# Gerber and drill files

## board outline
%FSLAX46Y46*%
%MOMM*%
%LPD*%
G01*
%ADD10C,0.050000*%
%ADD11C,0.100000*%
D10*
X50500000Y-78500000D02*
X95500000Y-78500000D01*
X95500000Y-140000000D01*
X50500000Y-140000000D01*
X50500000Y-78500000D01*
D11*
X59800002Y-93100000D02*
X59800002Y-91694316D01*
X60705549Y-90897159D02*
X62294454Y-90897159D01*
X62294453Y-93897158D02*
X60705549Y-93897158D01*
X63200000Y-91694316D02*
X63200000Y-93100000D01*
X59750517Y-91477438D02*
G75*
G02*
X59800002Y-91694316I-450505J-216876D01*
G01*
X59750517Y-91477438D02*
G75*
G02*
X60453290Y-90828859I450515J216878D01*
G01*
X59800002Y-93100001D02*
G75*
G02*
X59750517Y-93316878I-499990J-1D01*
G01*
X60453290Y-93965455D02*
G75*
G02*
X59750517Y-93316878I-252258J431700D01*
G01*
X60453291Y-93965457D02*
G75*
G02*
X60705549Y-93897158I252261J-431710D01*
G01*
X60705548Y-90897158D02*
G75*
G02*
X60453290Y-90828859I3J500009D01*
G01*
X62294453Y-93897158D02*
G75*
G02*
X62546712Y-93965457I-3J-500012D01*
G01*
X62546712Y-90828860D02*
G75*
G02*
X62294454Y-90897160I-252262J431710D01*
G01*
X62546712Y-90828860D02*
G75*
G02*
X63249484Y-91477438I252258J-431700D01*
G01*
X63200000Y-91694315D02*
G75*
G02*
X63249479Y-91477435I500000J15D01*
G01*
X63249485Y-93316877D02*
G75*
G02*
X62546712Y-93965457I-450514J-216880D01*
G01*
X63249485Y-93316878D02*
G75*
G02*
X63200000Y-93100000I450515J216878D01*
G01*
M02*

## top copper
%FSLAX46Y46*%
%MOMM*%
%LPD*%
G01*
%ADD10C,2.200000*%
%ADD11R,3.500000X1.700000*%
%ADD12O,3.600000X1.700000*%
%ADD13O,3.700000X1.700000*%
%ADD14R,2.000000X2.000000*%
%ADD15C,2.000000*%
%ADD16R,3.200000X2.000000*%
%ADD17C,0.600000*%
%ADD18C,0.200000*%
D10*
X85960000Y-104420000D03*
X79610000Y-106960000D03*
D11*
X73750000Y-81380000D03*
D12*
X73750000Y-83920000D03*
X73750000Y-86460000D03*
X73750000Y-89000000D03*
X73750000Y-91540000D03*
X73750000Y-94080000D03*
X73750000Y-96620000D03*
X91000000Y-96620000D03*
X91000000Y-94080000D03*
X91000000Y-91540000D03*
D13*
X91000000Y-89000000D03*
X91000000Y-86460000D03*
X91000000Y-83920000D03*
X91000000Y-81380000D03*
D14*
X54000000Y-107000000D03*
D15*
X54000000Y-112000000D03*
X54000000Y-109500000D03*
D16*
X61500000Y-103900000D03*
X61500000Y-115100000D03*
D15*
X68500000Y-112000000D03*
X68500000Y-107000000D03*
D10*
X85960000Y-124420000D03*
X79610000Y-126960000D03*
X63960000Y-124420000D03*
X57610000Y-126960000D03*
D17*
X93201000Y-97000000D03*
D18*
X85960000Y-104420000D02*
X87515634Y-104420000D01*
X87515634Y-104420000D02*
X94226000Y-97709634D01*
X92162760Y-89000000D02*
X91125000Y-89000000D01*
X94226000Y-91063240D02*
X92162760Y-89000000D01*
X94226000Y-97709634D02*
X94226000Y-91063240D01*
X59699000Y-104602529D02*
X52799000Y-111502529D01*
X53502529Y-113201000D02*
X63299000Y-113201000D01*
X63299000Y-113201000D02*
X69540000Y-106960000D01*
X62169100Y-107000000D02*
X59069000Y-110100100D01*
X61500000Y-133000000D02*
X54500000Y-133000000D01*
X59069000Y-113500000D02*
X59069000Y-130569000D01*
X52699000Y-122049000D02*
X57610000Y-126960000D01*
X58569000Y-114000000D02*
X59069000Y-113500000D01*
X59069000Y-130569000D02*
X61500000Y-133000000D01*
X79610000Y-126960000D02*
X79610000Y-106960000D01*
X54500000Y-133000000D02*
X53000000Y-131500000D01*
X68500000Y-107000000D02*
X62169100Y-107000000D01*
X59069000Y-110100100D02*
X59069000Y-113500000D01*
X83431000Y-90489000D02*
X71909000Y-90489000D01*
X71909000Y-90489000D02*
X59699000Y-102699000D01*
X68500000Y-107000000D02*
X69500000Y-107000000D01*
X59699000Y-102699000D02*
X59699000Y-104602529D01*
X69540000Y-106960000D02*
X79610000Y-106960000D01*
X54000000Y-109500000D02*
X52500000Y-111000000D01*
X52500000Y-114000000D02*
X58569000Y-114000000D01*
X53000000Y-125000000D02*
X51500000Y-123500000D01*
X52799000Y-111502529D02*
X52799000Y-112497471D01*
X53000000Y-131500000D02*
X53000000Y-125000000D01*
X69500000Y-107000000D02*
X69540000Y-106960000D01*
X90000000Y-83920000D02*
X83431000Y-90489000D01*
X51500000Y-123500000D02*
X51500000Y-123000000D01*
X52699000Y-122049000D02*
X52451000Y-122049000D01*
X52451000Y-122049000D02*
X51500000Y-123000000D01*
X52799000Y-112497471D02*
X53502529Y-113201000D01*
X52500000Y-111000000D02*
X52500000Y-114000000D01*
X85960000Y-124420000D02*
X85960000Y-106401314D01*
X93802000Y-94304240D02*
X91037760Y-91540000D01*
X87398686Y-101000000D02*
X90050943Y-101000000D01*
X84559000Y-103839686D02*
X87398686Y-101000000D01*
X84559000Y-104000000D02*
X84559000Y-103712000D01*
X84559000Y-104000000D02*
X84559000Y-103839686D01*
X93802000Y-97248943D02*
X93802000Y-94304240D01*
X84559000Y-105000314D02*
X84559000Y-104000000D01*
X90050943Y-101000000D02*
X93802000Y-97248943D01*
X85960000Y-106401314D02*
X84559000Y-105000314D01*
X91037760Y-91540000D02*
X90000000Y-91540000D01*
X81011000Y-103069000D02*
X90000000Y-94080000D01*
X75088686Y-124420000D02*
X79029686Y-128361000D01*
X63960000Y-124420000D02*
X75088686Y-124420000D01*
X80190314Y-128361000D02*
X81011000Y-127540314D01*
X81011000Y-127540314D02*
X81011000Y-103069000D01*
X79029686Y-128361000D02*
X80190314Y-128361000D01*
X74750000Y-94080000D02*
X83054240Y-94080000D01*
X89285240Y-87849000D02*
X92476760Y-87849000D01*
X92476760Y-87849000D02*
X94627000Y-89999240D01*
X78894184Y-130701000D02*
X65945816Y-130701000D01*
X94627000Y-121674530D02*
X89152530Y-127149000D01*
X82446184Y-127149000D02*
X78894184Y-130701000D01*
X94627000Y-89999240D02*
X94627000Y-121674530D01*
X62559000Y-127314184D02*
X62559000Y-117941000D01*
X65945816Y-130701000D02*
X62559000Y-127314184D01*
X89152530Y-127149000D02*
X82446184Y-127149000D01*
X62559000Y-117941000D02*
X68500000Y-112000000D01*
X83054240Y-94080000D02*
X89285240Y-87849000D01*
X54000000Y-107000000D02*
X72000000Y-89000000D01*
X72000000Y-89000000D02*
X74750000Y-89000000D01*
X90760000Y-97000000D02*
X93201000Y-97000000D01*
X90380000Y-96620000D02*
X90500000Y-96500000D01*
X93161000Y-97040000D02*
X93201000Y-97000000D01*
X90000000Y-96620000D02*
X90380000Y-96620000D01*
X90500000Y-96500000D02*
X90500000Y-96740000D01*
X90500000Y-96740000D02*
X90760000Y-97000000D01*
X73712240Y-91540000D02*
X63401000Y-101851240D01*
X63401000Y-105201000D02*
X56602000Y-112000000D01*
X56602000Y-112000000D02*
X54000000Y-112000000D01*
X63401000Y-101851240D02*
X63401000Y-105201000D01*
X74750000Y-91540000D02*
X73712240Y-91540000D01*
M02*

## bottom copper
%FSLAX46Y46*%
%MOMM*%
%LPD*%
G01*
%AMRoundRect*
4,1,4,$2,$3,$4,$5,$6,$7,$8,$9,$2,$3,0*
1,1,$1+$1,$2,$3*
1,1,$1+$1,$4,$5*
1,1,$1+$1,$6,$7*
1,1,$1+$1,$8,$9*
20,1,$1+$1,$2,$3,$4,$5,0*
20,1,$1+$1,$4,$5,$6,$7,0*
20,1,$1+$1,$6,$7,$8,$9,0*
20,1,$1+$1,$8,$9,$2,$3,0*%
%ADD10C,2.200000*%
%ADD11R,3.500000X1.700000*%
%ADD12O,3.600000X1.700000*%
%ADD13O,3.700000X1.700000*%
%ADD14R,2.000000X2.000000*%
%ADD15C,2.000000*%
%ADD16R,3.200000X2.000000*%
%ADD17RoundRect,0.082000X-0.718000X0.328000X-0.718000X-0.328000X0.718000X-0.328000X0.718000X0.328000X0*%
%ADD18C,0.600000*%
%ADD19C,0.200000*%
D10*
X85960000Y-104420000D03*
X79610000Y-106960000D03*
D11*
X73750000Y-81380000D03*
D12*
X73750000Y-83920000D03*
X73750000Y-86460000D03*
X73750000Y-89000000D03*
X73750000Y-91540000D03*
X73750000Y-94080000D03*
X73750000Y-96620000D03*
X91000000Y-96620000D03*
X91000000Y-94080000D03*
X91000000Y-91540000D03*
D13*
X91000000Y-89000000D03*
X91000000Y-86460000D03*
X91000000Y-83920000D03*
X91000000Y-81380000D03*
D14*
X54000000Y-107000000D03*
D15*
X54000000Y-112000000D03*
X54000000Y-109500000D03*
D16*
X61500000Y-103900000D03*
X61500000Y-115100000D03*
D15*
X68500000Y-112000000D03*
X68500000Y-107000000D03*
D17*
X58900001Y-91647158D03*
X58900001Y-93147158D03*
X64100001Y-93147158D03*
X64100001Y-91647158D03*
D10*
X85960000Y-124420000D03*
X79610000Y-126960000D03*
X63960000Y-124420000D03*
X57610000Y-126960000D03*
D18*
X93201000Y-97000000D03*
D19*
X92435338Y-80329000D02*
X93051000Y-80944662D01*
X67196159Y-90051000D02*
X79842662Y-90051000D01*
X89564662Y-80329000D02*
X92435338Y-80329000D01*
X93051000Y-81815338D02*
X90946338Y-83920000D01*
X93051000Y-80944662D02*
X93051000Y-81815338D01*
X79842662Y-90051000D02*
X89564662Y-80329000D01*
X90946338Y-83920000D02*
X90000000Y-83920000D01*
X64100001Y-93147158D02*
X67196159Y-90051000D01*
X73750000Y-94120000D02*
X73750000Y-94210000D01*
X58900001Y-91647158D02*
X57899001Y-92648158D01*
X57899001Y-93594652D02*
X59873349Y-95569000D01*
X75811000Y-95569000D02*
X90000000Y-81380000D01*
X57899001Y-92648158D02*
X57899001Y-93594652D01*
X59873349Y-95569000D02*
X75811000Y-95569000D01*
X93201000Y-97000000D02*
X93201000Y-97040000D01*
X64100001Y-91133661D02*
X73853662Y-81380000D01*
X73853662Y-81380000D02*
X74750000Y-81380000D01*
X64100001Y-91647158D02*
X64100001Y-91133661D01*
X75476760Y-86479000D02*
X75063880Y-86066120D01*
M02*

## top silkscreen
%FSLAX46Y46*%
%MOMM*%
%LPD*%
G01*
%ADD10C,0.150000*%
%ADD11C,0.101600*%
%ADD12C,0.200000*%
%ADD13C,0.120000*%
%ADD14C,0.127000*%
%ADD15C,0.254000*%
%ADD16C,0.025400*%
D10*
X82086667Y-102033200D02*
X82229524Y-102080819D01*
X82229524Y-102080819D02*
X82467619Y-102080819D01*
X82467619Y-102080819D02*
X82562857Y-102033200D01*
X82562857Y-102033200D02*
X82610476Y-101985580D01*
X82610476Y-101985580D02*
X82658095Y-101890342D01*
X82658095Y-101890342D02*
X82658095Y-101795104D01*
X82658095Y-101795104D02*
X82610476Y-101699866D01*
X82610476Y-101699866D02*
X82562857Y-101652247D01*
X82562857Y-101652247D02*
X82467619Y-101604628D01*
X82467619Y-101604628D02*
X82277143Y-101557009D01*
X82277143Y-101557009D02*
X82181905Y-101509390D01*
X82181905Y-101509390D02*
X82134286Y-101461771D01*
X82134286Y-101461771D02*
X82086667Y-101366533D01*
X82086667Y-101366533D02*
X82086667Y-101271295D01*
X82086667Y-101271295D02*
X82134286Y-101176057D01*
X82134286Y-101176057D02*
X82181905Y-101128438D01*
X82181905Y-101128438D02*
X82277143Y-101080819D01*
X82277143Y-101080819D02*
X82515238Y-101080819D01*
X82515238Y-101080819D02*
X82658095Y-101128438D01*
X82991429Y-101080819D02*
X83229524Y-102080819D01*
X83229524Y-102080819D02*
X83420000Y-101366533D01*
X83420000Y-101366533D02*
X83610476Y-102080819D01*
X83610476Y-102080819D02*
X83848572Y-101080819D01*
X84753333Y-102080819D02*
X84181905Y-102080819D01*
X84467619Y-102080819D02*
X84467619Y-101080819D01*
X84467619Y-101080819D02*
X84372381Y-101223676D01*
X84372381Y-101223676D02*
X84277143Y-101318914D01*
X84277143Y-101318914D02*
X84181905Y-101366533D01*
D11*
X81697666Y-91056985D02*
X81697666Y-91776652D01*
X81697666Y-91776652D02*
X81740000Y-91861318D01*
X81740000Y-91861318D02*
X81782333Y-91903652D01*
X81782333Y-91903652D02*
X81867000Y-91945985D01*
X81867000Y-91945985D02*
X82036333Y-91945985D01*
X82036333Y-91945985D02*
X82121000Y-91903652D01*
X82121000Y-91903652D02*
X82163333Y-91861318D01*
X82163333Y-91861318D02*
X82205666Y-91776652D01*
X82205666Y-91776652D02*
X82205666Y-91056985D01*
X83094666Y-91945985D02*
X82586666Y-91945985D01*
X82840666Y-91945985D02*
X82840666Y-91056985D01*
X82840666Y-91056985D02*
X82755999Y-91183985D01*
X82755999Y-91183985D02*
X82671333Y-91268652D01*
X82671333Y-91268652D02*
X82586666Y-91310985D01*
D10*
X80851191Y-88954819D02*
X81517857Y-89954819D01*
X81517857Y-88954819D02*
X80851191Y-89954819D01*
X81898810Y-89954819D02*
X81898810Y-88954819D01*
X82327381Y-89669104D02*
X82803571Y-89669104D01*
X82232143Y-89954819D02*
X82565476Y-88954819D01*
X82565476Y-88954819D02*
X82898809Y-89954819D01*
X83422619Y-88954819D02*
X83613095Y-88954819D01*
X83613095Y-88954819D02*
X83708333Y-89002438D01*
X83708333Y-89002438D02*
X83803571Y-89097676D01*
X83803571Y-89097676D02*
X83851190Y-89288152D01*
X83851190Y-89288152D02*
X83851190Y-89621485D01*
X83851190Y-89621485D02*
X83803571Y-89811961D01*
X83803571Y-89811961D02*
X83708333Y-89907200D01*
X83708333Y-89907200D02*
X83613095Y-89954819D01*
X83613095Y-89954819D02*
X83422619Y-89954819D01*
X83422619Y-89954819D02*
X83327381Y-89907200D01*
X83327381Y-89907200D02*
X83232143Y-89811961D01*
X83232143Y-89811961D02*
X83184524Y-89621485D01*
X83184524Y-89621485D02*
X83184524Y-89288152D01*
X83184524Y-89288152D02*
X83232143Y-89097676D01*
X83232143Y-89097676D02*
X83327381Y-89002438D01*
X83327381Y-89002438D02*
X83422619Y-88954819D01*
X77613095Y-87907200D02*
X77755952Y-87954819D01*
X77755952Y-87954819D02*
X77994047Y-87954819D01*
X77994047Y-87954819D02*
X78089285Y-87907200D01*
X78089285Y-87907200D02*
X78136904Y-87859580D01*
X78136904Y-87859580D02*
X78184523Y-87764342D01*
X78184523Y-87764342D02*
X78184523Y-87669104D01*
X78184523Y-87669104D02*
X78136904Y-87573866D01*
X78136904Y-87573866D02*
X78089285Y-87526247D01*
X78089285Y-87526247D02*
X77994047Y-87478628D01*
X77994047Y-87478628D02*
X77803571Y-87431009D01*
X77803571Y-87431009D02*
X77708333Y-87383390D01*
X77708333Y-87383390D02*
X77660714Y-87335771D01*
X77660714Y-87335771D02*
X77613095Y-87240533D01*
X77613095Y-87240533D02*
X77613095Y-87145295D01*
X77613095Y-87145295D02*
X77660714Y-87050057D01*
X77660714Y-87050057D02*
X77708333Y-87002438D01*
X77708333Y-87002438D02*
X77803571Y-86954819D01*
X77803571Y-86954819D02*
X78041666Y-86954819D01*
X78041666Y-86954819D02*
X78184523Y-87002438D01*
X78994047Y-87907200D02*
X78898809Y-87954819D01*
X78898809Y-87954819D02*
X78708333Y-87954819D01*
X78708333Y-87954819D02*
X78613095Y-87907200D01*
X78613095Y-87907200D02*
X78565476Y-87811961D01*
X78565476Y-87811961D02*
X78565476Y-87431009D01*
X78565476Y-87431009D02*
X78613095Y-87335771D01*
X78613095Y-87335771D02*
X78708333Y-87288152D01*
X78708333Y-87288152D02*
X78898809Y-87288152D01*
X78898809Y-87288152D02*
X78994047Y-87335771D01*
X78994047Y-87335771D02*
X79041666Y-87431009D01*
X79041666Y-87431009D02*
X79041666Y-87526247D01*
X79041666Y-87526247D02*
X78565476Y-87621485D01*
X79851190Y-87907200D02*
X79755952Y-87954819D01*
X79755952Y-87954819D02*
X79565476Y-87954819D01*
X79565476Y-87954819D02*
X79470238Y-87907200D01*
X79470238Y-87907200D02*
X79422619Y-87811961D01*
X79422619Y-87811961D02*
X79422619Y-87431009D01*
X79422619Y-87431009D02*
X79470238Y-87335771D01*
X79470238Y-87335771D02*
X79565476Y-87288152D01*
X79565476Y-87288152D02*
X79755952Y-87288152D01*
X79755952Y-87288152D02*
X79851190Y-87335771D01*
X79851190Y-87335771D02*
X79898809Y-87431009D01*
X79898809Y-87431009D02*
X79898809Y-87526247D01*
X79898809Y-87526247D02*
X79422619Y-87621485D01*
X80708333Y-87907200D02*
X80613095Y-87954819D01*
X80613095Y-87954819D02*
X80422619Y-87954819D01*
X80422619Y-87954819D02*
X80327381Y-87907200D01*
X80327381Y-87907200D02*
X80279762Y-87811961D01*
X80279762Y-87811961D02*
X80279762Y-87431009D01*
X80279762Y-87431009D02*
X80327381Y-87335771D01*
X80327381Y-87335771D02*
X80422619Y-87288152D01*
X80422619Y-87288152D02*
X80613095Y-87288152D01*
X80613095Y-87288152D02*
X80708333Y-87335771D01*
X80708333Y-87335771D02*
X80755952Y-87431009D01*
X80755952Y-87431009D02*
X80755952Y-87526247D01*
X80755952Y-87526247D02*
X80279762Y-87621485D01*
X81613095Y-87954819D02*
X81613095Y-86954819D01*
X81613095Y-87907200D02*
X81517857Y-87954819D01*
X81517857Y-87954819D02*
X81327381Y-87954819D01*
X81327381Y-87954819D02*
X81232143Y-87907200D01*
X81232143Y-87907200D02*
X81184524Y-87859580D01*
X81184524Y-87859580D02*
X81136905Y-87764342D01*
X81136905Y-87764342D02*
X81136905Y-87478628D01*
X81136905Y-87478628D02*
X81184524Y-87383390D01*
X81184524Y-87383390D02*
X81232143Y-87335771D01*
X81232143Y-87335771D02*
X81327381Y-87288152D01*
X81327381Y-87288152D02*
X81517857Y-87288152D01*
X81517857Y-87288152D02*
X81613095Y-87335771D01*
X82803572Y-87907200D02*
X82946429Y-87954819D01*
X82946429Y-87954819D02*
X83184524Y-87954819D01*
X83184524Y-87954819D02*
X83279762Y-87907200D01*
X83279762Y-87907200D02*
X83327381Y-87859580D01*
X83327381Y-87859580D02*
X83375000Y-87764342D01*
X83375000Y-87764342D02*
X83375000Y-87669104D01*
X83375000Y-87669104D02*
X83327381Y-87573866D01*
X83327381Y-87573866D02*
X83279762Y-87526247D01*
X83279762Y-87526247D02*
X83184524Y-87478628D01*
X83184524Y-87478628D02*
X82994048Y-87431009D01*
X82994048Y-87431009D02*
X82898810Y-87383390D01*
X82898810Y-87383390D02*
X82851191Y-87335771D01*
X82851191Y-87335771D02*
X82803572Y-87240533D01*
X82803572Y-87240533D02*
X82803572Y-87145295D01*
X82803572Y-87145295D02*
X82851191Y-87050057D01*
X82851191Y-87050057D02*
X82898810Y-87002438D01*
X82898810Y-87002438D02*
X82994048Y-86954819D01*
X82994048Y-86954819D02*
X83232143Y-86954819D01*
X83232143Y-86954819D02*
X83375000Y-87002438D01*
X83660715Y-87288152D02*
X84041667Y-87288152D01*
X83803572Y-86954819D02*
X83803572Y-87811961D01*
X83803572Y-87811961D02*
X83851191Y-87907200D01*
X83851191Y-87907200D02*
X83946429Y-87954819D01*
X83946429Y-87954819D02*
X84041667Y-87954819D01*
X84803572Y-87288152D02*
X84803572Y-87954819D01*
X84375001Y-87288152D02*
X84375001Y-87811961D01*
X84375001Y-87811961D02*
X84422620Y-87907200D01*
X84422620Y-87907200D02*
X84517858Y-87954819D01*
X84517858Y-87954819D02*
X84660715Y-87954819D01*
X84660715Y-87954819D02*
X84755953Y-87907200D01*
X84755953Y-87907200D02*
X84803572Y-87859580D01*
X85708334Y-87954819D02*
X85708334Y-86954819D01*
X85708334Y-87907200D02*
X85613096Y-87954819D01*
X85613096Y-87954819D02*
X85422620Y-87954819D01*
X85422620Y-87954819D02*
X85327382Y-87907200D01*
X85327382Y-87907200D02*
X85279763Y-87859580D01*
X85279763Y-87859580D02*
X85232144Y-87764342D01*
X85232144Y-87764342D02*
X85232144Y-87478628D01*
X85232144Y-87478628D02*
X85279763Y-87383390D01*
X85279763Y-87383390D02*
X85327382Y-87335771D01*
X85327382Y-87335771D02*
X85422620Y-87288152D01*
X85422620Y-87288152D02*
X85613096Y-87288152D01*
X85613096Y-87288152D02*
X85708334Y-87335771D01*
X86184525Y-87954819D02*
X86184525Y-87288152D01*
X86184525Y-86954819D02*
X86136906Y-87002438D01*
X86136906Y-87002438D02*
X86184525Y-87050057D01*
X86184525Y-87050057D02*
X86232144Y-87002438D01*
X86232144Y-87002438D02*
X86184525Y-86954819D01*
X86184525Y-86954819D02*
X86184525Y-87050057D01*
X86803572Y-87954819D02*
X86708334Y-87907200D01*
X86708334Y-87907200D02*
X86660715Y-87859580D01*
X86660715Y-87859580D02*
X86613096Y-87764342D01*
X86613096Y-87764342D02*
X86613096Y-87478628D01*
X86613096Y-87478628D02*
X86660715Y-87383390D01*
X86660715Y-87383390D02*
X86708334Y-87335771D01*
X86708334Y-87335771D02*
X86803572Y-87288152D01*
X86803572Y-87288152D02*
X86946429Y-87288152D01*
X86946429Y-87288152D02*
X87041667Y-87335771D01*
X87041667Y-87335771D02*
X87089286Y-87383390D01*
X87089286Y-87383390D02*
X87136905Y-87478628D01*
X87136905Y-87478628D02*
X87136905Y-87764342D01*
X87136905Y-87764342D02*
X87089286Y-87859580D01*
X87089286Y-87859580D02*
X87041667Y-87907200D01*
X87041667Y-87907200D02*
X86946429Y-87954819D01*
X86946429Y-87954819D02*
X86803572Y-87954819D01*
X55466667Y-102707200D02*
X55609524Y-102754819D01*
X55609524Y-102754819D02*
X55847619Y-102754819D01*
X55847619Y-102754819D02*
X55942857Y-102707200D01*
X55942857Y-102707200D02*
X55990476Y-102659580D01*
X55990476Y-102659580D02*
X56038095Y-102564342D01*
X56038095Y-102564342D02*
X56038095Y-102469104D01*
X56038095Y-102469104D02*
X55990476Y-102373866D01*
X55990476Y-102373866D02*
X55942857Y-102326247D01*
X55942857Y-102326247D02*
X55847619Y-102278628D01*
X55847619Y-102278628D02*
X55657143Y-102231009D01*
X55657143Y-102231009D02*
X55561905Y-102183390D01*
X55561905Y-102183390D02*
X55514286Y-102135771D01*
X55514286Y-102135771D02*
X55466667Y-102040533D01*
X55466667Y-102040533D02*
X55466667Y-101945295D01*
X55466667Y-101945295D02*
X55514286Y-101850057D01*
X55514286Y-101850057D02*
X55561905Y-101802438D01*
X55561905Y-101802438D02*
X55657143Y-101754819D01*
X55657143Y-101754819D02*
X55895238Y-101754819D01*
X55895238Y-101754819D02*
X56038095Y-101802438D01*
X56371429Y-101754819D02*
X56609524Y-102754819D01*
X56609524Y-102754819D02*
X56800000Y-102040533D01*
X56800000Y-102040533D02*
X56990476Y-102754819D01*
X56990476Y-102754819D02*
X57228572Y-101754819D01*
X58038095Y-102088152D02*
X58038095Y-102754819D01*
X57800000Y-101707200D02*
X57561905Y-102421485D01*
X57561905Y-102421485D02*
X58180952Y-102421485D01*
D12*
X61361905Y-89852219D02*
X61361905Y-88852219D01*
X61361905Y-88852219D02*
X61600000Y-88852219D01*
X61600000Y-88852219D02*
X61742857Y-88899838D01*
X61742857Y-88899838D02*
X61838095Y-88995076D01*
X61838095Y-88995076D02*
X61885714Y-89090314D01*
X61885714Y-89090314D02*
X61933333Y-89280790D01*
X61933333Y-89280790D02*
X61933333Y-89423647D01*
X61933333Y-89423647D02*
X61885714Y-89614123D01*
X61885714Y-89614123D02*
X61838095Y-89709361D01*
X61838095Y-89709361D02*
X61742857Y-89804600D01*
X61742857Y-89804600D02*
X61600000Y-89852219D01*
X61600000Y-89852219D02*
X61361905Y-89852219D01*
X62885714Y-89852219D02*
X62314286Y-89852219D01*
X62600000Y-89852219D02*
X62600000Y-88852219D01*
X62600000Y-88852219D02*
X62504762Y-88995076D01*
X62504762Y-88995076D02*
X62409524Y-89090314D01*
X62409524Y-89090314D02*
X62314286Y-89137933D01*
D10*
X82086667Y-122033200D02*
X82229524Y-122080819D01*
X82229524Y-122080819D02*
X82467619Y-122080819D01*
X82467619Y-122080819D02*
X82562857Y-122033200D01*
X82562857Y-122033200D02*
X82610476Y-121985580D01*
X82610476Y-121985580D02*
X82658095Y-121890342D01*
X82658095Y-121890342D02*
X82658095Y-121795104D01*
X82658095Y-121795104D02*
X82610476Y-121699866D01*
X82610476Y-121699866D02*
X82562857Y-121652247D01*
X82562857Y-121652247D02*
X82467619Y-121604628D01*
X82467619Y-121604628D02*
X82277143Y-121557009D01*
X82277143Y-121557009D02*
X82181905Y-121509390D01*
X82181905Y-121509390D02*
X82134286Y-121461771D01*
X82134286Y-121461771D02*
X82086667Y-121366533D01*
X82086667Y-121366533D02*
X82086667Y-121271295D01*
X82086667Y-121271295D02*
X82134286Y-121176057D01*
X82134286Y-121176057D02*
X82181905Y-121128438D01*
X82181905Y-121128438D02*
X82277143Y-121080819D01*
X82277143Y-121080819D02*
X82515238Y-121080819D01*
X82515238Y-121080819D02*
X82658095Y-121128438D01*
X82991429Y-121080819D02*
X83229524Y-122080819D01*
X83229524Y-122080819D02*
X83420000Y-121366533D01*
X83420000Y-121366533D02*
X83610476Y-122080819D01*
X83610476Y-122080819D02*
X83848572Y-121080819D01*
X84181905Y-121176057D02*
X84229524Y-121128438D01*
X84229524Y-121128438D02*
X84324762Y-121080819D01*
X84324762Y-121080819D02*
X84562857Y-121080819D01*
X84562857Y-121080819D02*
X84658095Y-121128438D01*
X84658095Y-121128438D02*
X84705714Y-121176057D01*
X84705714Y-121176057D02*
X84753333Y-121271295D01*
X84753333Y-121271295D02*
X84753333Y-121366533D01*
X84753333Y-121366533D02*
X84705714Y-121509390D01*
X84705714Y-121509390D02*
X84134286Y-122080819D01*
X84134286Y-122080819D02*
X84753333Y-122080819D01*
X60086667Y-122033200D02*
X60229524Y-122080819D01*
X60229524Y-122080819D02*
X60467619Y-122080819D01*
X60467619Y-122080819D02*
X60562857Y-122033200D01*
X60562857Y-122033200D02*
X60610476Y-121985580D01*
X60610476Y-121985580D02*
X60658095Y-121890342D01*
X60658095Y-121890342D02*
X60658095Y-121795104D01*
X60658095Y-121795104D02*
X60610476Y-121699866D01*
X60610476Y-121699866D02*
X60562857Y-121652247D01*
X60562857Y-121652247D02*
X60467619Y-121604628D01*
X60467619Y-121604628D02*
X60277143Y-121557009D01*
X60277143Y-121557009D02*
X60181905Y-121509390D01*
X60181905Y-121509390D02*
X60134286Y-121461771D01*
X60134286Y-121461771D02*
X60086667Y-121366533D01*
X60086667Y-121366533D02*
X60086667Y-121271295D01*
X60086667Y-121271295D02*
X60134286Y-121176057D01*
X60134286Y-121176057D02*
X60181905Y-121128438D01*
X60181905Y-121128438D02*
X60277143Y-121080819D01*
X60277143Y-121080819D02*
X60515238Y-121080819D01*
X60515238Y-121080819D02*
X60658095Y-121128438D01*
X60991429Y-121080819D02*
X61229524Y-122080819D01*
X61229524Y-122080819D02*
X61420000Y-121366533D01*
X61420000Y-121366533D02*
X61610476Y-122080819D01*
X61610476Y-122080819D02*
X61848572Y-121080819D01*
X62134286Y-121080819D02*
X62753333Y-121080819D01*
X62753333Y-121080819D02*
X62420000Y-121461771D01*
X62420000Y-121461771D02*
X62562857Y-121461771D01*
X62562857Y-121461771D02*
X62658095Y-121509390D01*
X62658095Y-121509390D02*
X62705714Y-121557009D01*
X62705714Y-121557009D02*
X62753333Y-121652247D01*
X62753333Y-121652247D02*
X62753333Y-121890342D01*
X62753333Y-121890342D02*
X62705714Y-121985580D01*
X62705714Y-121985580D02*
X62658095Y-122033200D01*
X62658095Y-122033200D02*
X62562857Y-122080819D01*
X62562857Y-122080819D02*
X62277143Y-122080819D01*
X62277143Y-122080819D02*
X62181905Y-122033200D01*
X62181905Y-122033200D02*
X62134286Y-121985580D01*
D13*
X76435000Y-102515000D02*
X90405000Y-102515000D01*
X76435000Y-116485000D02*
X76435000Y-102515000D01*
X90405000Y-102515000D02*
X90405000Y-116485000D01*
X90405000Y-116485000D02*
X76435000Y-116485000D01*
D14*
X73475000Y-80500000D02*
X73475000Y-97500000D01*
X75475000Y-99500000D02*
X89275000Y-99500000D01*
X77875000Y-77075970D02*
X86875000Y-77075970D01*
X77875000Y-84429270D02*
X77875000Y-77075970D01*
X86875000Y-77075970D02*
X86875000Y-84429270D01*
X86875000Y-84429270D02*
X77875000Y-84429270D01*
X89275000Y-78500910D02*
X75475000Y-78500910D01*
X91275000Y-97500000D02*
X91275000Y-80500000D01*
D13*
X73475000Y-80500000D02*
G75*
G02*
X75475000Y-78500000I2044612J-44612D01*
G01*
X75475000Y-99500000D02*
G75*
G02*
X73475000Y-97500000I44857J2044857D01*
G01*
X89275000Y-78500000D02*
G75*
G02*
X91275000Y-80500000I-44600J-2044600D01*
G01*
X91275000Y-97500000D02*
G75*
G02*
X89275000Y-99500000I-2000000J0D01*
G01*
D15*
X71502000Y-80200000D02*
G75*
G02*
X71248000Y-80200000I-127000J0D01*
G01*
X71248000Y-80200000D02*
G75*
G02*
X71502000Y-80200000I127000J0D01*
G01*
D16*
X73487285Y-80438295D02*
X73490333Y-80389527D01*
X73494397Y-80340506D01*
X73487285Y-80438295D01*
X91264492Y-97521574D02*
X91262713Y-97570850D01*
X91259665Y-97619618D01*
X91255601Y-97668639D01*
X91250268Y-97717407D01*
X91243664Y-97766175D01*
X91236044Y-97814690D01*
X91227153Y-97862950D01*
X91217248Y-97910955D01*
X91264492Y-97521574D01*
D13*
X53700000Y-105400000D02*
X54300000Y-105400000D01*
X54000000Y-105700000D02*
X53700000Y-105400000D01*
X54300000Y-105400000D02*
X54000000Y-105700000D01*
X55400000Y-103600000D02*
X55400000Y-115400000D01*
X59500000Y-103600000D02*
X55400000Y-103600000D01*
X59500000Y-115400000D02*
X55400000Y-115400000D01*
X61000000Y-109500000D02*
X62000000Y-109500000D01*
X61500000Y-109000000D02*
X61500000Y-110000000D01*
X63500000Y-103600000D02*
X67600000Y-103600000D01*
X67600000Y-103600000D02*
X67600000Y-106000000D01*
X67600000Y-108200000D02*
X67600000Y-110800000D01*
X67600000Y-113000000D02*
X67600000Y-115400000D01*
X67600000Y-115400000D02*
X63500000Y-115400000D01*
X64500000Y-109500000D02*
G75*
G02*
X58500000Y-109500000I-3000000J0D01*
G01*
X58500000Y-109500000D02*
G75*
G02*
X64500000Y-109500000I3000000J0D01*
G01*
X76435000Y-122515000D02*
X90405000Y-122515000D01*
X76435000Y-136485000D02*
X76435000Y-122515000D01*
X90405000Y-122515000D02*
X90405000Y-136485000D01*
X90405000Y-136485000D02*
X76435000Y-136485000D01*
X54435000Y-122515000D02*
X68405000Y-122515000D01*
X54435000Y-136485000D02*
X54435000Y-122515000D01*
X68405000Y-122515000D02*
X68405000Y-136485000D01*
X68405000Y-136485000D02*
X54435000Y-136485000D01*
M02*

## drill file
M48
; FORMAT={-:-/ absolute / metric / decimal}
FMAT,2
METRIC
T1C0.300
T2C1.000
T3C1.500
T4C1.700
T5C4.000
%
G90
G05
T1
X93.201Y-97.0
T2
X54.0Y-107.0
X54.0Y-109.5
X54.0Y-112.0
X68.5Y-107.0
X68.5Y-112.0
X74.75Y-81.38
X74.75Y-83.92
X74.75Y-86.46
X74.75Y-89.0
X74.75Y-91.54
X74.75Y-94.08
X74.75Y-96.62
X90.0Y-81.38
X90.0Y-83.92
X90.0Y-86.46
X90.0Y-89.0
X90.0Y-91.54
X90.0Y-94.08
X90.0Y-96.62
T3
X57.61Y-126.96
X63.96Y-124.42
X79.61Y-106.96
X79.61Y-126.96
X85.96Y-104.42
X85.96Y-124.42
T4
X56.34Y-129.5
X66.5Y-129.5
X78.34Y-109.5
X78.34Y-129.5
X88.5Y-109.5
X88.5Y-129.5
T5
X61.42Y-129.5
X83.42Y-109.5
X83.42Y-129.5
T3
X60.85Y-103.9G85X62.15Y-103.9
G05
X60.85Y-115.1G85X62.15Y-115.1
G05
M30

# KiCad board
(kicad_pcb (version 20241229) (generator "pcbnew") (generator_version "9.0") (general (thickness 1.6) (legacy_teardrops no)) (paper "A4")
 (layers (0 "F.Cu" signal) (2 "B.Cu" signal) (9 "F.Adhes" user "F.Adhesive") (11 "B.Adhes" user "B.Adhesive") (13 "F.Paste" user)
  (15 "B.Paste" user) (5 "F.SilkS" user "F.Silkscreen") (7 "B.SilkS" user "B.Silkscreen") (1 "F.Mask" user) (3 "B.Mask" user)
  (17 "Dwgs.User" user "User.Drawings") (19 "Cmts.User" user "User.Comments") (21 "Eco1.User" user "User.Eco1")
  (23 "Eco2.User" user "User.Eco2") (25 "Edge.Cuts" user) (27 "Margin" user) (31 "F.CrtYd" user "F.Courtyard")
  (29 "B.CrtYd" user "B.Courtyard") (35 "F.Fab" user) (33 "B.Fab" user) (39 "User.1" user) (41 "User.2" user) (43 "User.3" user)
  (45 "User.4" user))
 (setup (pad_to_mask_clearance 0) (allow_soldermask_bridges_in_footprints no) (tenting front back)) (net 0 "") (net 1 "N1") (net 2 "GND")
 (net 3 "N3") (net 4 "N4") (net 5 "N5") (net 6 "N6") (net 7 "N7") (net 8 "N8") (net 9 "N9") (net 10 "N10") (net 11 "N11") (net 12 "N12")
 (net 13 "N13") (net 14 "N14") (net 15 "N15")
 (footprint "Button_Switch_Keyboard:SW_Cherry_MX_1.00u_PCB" (layer "F.Cu") (at 85.96 104.42)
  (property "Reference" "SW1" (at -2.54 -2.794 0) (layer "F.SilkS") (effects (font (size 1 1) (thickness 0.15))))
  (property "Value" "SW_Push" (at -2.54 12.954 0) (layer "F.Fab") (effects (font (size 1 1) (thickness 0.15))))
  (fp_line (start -9.525 -1.905) (end 4.445 -1.905) (stroke (width 0.12) (type solid)) (layer "F.SilkS"))
  (fp_line (start -9.525 12.065) (end -9.525 -1.905) (stroke (width 0.12) (type solid)) (layer "F.SilkS"))
  (fp_line (start 4.445 -1.905) (end 4.445 12.065) (stroke (width 0.12) (type solid)) (layer "F.SilkS"))
  (fp_line (start 4.445 12.065) (end -9.525 12.065) (stroke (width 0.12) (type solid)) (layer "F.SilkS"))
  (pad "" np_thru_hole circle (at -7.62 5.08) (size 1.7 1.7) (drill 1.7) (layers "*.Cu" "*.Mask"))
  (pad "" np_thru_hole circle (at -2.54 5.08) (size 4 4) (drill 4) (layers "*.Cu" "*.Mask"))
  (pad "" np_thru_hole circle (at 2.54 5.08) (size 1.7 1.7) (drill 1.7) (layers "*.Cu" "*.Mask"))
  (pad "1" thru_hole circle (at 0 0) (size 2.2 2.2) (drill 1.5) (layers "*.Cu" "*.Mask") (remove_unused_layers no) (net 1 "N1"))
  (pad "2" thru_hole circle (at -6.35 2.54) (size 2.2 2.2) (drill 1.5) (layers "*.Cu" "*.Mask") (remove_unused_layers no) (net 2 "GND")))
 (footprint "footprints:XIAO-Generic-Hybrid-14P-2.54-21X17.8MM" (layer "F.Cu") (at 82.375 89)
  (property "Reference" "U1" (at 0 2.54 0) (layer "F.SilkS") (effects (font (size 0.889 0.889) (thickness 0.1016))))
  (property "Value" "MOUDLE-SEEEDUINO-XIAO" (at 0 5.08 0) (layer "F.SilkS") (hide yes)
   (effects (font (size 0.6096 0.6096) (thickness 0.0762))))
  (fp_line (start -8.9 -8.5) (end -8.9 8.5) (stroke (width 0.127) (type solid)) (layer "F.SilkS"))
  (fp_line (start -6.9 10.5) (end 6.9 10.5) (stroke (width 0.127) (type solid)) (layer "F.SilkS"))
  (fp_line (start -4.5 -11.92403) (end 4.5 -11.92403) (stroke (width 0.127) (type solid)) (layer "F.SilkS"))
  (fp_line (start -4.5 -4.57073) (end -4.5 -11.92403) (stroke (width 0.127) (type solid)) (layer "F.SilkS"))
  (fp_line (start 4.5 -11.92403) (end 4.5 -4.57073) (stroke (width 0.127) (type solid)) (layer "F.SilkS"))
  (fp_line (start 4.5 -4.57073) (end -4.5 -4.57073) (stroke (width 0.127) (type solid)) (layer "F.SilkS"))
  (fp_line (start 6.9 -10.49909) (end -6.9 -10.49909) (stroke (width 0.127) (type solid)) (layer "F.SilkS"))
  (fp_line (start 8.9 8.5) (end 8.9 -8.5) (stroke (width 0.127) (type solid)) (layer "F.SilkS"))
  (fp_arc (start -8.9 -8.5) (mid -8.301491 -9.901491) (end -6.9 -10.5) (stroke (width 0.12) (type solid)) (layer "F.SilkS"))
  (fp_arc (start -6.9 10.5) (mid -8.301423 9.901423) (end -8.9 8.5) (stroke (width 0.12) (type solid)) (layer "F.SilkS"))
  (fp_arc (start 6.9 -10.5) (mid 8.301492 -9.901492) (end 8.9 -8.5) (stroke (width 0.12) (type solid)) (layer "F.SilkS"))
  (fp_arc (start 8.9 8.5) (mid 8.314214 9.914214) (end 6.9 10.5) (stroke (width 0.12) (type solid)) (layer "F.SilkS"))
  (fp_circle (center -11 -8.8) (end -11 -9.054) (stroke (width 0) (type solid)) (fill yes) (layer "F.SilkS"))
  (fp_poly
   (pts (xy -8.887715 -8.561705) (xy -8.884667 -8.610473) (xy -8.880603 -8.659494)) (stroke (width 0.0254) (type solid)) (fill no)
   (layer "F.SilkS"))
  (fp_poly
   (pts (xy 8.889492 8.521574) (xy 8.887713 8.57085) (xy 8.884665 8.619618) (xy 8.880601 8.668639) (xy 8.875268 8.717407)
    (xy 8.868664 8.766175) (xy 8.861044 8.81469) (xy 8.852153 8.86295) (xy 8.842248 8.910955))
   (stroke (width 0.0254) (type solid)) (fill no) (layer "F.SilkS"))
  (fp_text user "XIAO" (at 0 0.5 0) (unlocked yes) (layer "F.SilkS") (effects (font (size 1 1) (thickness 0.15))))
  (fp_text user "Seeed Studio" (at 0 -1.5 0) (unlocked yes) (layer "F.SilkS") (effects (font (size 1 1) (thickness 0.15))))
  (pad "1" thru_hole rect (at -7.625 -7.62) (size 3.5 1.7) (drill 1 (offset -1 0)) (layers "*.Cu" "*.Mask") (remove_unused_layers no)
   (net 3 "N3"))
  (pad "2" thru_hole oval (at -7.625 -5.08) (size 3.6 1.7) (drill 1 (offset -1 0)) (layers "*.Cu" "*.Mask") (remove_unused_layers no)
   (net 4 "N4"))
  (pad "3" thru_hole oval (at -7.625 -2.54) (size 3.6 1.7) (drill 1 (offset -1 0)) (layers "*.Cu" "*.Mask") (remove_unused_layers no)
   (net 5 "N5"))
  (pad "4" thru_hole oval (at -7.625 0) (size 3.6 1.7) (drill 1 (offset -1 0)) (layers "*.Cu" "*.Mask") (remove_unused_layers no)
   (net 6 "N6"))
  (pad "5" thru_hole oval (at -7.625 2.54) (size 3.6 1.7) (drill 1 (offset -1 0)) (layers "*.Cu" "*.Mask") (remove_unused_layers no)
   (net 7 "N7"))
  (pad "6" thru_hole oval (at -7.625 5.08 180) (size 3.6 1.7) (drill 1 (offset 1 0)) (layers "*.Cu" "*.Mask") (remove_unused_layers no)
   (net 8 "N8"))
  (pad "7" thru_hole oval (at -7.625 7.62) (size 3.6 1.7) (drill 1 (offset -1 0)) (layers "*.Cu" "*.Mask") (remove_unused_layers no)
   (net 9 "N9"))
  (pad "8" thru_hole oval (at 7.625 7.62) (size 3.6 1.7) (drill 1 (offset 1 0)) (layers "*.Cu" "*.Mask") (remove_unused_layers no)
   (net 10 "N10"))
  (pad "9" thru_hole oval (at 7.625 5.08) (size 3.6 1.7) (drill 1 (offset 1 0)) (layers "*.Cu" "*.Mask") (remove_unused_layers no)
   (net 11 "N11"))
  (pad "10" thru_hole oval (at 7.625 2.54) (size 3.6 1.7) (drill 1 (offset 1 0)) (layers "*.Cu" "*.Mask") (remove_unused_layers no)
   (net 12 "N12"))
  (pad "11" thru_hole oval (at 7.625 0) (size 3.7 1.7) (drill 1 (offset 1 0)) (layers "*.Cu" "*.Mask") (remove_unused_layers no)
   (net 1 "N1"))
  (pad "12" thru_hole oval (at 7.625 -2.54) (size 3.7 1.7) (drill 1 (offset 1 0)) (layers "*.Cu" "*.Mask") (remove_unused_layers no)
   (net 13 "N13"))
  (pad "13" thru_hole oval (at 7.625 -5.08) (size 3.7 1.7) (drill 1 (offset 1 0)) (layers "*.Cu" "*.Mask") (remove_unused_layers no)
   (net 2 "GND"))
  (pad "14" thru_hole oval (at 7.625 -7.62) (size 3.7 1.7) (drill 1 (offset 1 0)) (layers "*.Cu" "*.Mask") (remove_unused_layers no)
   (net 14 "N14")))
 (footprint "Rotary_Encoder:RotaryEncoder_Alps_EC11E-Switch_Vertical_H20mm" (layer "F.Cu") (at 54 107)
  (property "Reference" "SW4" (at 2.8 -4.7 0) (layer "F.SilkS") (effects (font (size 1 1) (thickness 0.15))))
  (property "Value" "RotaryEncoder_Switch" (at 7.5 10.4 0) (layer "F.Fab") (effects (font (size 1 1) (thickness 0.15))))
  (fp_line (start -0.3 -1.6) (end 0.3 -1.6) (stroke (width 0.12) (type solid)) (layer "F.SilkS"))
  (fp_line (start 0 -1.3) (end -0.3 -1.6) (stroke (width 0.12) (type solid)) (layer "F.SilkS"))
  (fp_line (start 0.3 -1.6) (end 0 -1.3) (stroke (width 0.12) (type solid)) (layer "F.SilkS"))
  (fp_line (start 1.4 -3.4) (end 1.4 8.4) (stroke (width 0.12) (type solid)) (layer "F.SilkS"))
  (fp_line (start 5.5 -3.4) (end 1.4 -3.4) (stroke (width 0.12) (type solid)) (layer "F.SilkS"))
  (fp_line (start 5.5 8.4) (end 1.4 8.4) (stroke (width 0.12) (type solid)) (layer "F.SilkS"))
  (fp_line (start 7 2.5) (end 8 2.5) (stroke (width 0.12) (type solid)) (layer "F.SilkS"))
  (fp_line (start 7.5 2) (end 7.5 3) (stroke (width 0.12) (type solid)) (layer "F.SilkS"))
  (fp_line (start 9.5 -3.4) (end 13.6 -3.4) (stroke (width 0.12) (type solid)) (layer "F.SilkS"))
  (fp_line (start 13.6 -3.4) (end 13.6 -1) (stroke (width 0.12) (type solid)) (layer "F.SilkS"))
  (fp_line (start 13.6 1.2) (end 13.6 3.8) (stroke (width 0.12) (type solid)) (layer "F.SilkS"))
  (fp_line (start 13.6 6) (end 13.6 8.4) (stroke (width 0.12) (type solid)) (layer "F.SilkS"))
  (fp_line (start 13.6 8.4) (end 9.5 8.4) (stroke (width 0.12) (type solid)) (layer "F.SilkS"))
  (fp_circle (center 7.5 2.5) (end 10.5 2.5) (stroke (width 0.12) (type solid)) (fill no) (layer "F.SilkS"))
  (pad "A" thru_hole rect (at 0 0) (size 2 2) (drill 1) (layers "*.Cu" "*.Mask") (remove_unused_layers no) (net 6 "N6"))
  (pad "B" thru_hole circle (at 0 5) (size 2 2) (drill 1) (layers "*.Cu" "*.Mask") (remove_unused_layers no) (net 7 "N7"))
  (pad "C" thru_hole circle (at 0 2.5) (size 2 2) (drill 1) (layers "*.Cu" "*.Mask") (remove_unused_layers no) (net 2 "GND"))
  (pad "MP" thru_hole rect (at 7.5 -3.1) (size 3.2 2) (drill oval 2.8 1.5) (layers "*.Cu" "*.Mask") (remove_unused_layers no))
  (pad "MP" thru_hole rect (at 7.5 8.1) (size 3.2 2) (drill oval 2.8 1.5) (layers "*.Cu" "*.Mask") (remove_unused_layers no))
  (pad "S1" thru_hole circle (at 14.5 5) (size 2 2) (drill 1) (layers "*.Cu" "*.Mask") (remove_unused_layers no) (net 8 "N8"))
  (pad "S2" thru_hole circle (at 14.5 0) (size 2 2) (drill 1) (layers "*.Cu" "*.Mask") (remove_unused_layers no) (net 2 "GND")))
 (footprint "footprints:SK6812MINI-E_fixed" (layer "F.Cu") (at 61.5 92.5)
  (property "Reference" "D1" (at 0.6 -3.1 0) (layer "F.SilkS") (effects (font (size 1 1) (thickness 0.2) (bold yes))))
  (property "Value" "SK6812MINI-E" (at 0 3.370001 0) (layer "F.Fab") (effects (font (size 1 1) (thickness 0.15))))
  (fp_line (start -1.699998 0.6) (end -1.699998 -0.805684) (stroke (width 0.1) (type solid)) (layer "Edge.Cuts"))
  (fp_line (start -0.794451 -1.602841) (end 0.794454 -1.602841) (stroke (width 0.1) (type solid)) (layer "Edge.Cuts"))
  (fp_line (start 0.794453 1.397158) (end -0.794451 1.397158) (stroke (width 0.1) (type solid)) (layer "Edge.Cuts"))
  (fp_line (start 1.7 -0.805684) (end 1.7 0.6) (stroke (width 0.1) (type solid)) (layer "Edge.Cuts"))
  (fp_arc (start -1.749483 -1.022562) (mid -1.712526 -0.91691) (end -1.699998 -0.805684) (stroke (width 0.1) (type solid))
   (layer "Edge.Cuts"))
  (fp_arc (start -1.749483 -1.022562) (mid -1.63807 -1.606877) (end -1.04671 -1.671141) (stroke (width 0.1) (type solid))
   (layer "Edge.Cuts"))
  (fp_arc (start -1.699998 0.600001) (mid -1.712526 0.711226) (end -1.749483 0.816878) (stroke (width 0.1) (type solid)) (layer "Edge.Cuts"))
  (fp_arc (start -1.04671 1.465455) (mid -1.638069 1.401192) (end -1.749483 0.816878) (stroke (width 0.1) (type solid)) (layer "Edge.Cuts"))
  (fp_arc (start -1.046709 1.465457) (mid -0.925121 1.414535) (end -0.794451 1.397158) (stroke (width 0.1) (type solid)) (layer "Edge.Cuts"))
  (fp_arc (start -0.794452 -1.602842) (mid -0.925122 -1.620219) (end -1.04671 -1.671141) (stroke (width 0.1) (type solid))
   (layer "Edge.Cuts"))
  (fp_arc (start 0.794453 1.397158) (mid 0.925124 1.414535) (end 1.046712 1.465457) (stroke (width 0.1) (type solid)) (layer "Edge.Cuts"))
  (fp_arc (start 1.046712 -1.67114) (mid 0.925124 -1.620218) (end 0.794454 -1.602841) (stroke (width 0.1) (type solid)) (layer "Edge.Cuts"))
  (fp_arc (start 1.046712 -1.67114) (mid 1.638072 -1.606876) (end 1.749485 -1.022562) (stroke (width 0.1) (type solid)) (layer "Edge.Cuts"))
  (fp_arc (start 1.7 -0.805685) (mid 1.712528 -0.91691) (end 1.749485 -1.022562) (stroke (width 0.1) (type solid)) (layer "Edge.Cuts"))
  (fp_arc (start 1.749485 0.816877) (mid 1.638073 1.401193) (end 1.046712 1.465457) (stroke (width 0.1) (type solid)) (layer "Edge.Cuts"))
  (fp_arc (start 1.749485 0.816878) (mid 1.712528 0.711226) (end 1.7 0.6) (stroke (width 0.1) (type solid)) (layer "Edge.Cuts"))
  (pad "1" smd roundrect (at -2.599999 -0.852842 270) (size 0.82 1.6) (layers "B.Cu" "B.Mask" "B.Paste") (roundrect_rratio 0.1)
   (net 14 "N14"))
  (pad "2" smd roundrect (at -2.599999 0.647158 270) (size 0.82 1.6) (layers "B.Cu" "B.Mask" "B.Paste") (roundrect_rratio 0.1)
   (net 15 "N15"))
  (pad "3" smd roundrect (at 2.600001 0.647158 270) (size 0.82 1.6) (layers "B.Cu" "B.Mask" "B.Paste") (roundrect_rratio 0.1) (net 2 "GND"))
  (pad "4" smd roundrect (at 2.600001 -0.852842 270) (size 0.82 1.6) (layers "B.Cu" "B.Mask" "B.Paste") (roundrect_rratio 0.1) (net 3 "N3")))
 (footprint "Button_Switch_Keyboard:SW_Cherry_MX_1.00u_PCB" (layer "F.Cu") (at 85.96 124.42)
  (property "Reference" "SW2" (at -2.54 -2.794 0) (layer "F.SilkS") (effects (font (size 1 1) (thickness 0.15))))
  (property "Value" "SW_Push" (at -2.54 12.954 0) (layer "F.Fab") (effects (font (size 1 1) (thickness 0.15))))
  (fp_line (start -9.525 -1.905) (end 4.445 -1.905) (stroke (width 0.12) (type solid)) (layer "F.SilkS"))
  (fp_line (start -9.525 12.065) (end -9.525 -1.905) (stroke (width 0.12) (type solid)) (layer "F.SilkS"))
  (fp_line (start 4.445 -1.905) (end 4.445 12.065) (stroke (width 0.12) (type solid)) (layer "F.SilkS"))
  (fp_line (start 4.445 12.065) (end -9.525 12.065) (stroke (width 0.12) (type solid)) (layer "F.SilkS"))
  (pad "" np_thru_hole circle (at -7.62 5.08) (size 1.7 1.7) (drill 1.7) (layers "*.Cu" "*.Mask"))
  (pad "" np_thru_hole circle (at -2.54 5.08) (size 4 4) (drill 4) (layers "*.Cu" "*.Mask"))
  (pad "" np_thru_hole circle (at 2.54 5.08) (size 1.7 1.7) (drill 1.7) (layers "*.Cu" "*.Mask"))
  (pad "1" thru_hole circle (at 0 0) (size 2.2 2.2) (drill 1.5) (layers "*.Cu" "*.Mask") (remove_unused_layers no) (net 12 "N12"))
  (pad "2" thru_hole circle (at -6.35 2.54) (size 2.2 2.2) (drill 1.5) (layers "*.Cu" "*.Mask") (remove_unused_layers no) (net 2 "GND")))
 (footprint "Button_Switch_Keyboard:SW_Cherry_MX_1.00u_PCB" (layer "F.Cu") (at 63.96 124.42)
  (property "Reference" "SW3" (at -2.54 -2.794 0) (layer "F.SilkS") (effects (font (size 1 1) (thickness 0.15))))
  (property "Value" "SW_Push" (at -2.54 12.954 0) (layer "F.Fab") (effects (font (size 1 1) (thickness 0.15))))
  (fp_line (start -9.525 -1.905) (end 4.445 -1.905) (stroke (width 0.12) (type solid)) (layer "F.SilkS"))
  (fp_line (start -9.525 12.065) (end -9.525 -1.905) (stroke (width 0.12) (type solid)) (layer "F.SilkS"))
  (fp_line (start 4.445 -1.905) (end 4.445 12.065) (stroke (width 0.12) (type solid)) (layer "F.SilkS"))
  (fp_line (start 4.445 12.065) (end -9.525 12.065) (stroke (width 0.12) (type solid)) (layer "F.SilkS"))
  (pad "" np_thru_hole circle (at -7.62 5.08) (size 1.7 1.7) (drill 1.7) (layers "*.Cu" "*.Mask"))
  (pad "" np_thru_hole circle (at -2.54 5.08) (size 4 4) (drill 4) (layers "*.Cu" "*.Mask"))
  (pad "" np_thru_hole circle (at 2.54 5.08) (size 1.7 1.7) (drill 1.7) (layers "*.Cu" "*.Mask"))
  (pad "1" thru_hole circle (at 0 0) (size 2.2 2.2) (drill 1.5) (layers "*.Cu" "*.Mask") (remove_unused_layers no) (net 11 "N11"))
  (pad "2" thru_hole circle (at -6.35 2.54) (size 2.2 2.2) (drill 1.5) (layers "*.Cu" "*.Mask") (remove_unused_layers no) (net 2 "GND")))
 (gr_rect (start 50.5 78.5) (end 95.5 140) (stroke (width 0.05) (type default)) (fill no) (layer "Edge.Cuts"))
 (segment (start 85.96 104.42) (end 87.515634 104.42) (width 0.2) (layer "F.Cu") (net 1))
 (segment (start 87.515634 104.42) (end 94.226 97.709634) (width 0.2) (layer "F.Cu") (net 1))
 (segment (start 92.16276 89) (end 91.125 89) (width 0.2) (layer "F.Cu") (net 1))
 (segment (start 94.226 91.06324) (end 92.16276 89) (width 0.2) (layer "F.Cu") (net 1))
 (segment (start 94.226 97.709634) (end 94.226 91.06324) (width 0.2) (layer "F.Cu") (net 1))
 (segment (start 59.699 104.602529) (end 52.799 111.502529) (width 0.2) (layer "F.Cu") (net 2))
 (segment (start 53.502529 113.201) (end 63.299 113.201) (width 0.2) (layer "F.Cu") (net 2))
 (segment (start 63.299 113.201) (end 69.54 106.96) (width 0.2) (layer "F.Cu") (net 2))
 (segment (start 62.1691 107) (end 59.069 110.1001) (width 0.2) (layer "F.Cu") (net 2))
 (segment (start 61.5 133) (end 54.5 133) (width 0.2) (layer "F.Cu") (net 2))
 (segment (start 59.069 113.5) (end 59.069 130.569) (width 0.2) (layer "F.Cu") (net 2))
 (segment (start 52.699 122.049) (end 57.61 126.96) (width 0.2) (layer "F.Cu") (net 2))
 (segment (start 58.569 114) (end 59.069 113.5) (width 0.2) (layer "F.Cu") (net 2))
 (segment (start 59.069 130.569) (end 61.5 133) (width 0.2) (layer "F.Cu") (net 2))
 (segment (start 79.61 126.96) (end 79.61 106.96) (width 0.2) (layer "F.Cu") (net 2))
 (segment (start 54.5 133) (end 53 131.5) (width 0.2) (layer "F.Cu") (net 2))
 (segment (start 68.5 107) (end 62.1691 107) (width 0.2) (layer "F.Cu") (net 2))
 (segment (start 59.069 110.1001) (end 59.069 113.5) (width 0.2) (layer "F.Cu") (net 2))
 (segment (start 83.431 90.489) (end 71.909 90.489) (width 0.2) (layer "F.Cu") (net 2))
 (segment (start 71.909 90.489) (end 59.699 102.699) (width 0.2) (layer "F.Cu") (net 2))
 (segment (start 68.5 107) (end 69.5 107) (width 0.2) (layer "F.Cu") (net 2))
 (segment (start 59.699 102.699) (end 59.699 104.602529) (width 0.2) (layer "F.Cu") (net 2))
 (segment (start 69.54 106.96) (end 79.61 106.96) (width 0.2) (layer "F.Cu") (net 2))
 (segment (start 54 109.5) (end 52.5 111) (width 0.2) (layer "F.Cu") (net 2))
 (segment (start 52.5 114) (end 58.569 114) (width 0.2) (layer "F.Cu") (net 2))
 (segment (start 53 125) (end 51.5 123.5) (width 0.2) (layer "F.Cu") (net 2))
 (segment (start 52.799 111.502529) (end 52.799 112.497471) (width 0.2) (layer "F.Cu") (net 2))
 (segment (start 53 131.5) (end 53 125) (width 0.2) (layer "F.Cu") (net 2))
 (segment (start 69.5 107) (end 69.54 106.96) (width 0.2) (layer "F.Cu") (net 2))
 (segment (start 90 83.92) (end 83.431 90.489) (width 0.2) (layer "F.Cu") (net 2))
 (segment (start 51.5 123.5) (end 51.5 123) (width 0.2) (layer "F.Cu") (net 2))
 (segment (start 52.699 122.049) (end 52.451 122.049) (width 0.2) (layer "F.Cu") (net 2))
 (segment (start 52.451 122.049) (end 51.5 123) (width 0.2) (layer "F.Cu") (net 2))
 (segment (start 52.799 112.497471) (end 53.502529 113.201) (width 0.2) (layer "F.Cu") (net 2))
 (segment (start 52.5 111) (end 52.5 114) (width 0.2) (layer "F.Cu") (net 2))
 (segment (start 92.435338 80.329) (end 93.051 80.944662) (width 0.2) (layer "B.Cu") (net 2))
 (segment (start 67.196159 90.051) (end 79.842662 90.051) (width 0.2) (layer "B.Cu") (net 2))
 (segment (start 89.564662 80.329) (end 92.435338 80.329) (width 0.2) (layer "B.Cu") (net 2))
 (segment (start 93.051 81.815338) (end 90.946338 83.92) (width 0.2) (layer "B.Cu") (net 2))
 (segment (start 93.051 80.944662) (end 93.051 81.815338) (width 0.2) (layer "B.Cu") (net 2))
 (segment (start 79.842662 90.051) (end 89.564662 80.329) (width 0.2) (layer "B.Cu") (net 2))
 (segment (start 90.946338 83.92) (end 90 83.92) (width 0.2) (layer "B.Cu") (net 2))
 (segment (start 64.100001 93.147158) (end 67.196159 90.051) (width 0.2) (layer "B.Cu") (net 2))
 (segment (start 85.96 124.42) (end 85.96 106.401314) (width 0.2) (layer "F.Cu") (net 12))
 (segment (start 93.802 94.30424) (end 91.03776 91.54) (width 0.2) (layer "F.Cu") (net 12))
 (segment (start 87.398686 101) (end 90.050943 101) (width 0.2) (layer "F.Cu") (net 12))
 (segment (start 84.559 103.839686) (end 87.398686 101) (width 0.2) (layer "F.Cu") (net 12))
 (segment (start 84.559 104) (end 84.559 103.712) (width 0.2) (layer "F.Cu") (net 12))
 (segment (start 84.559 104) (end 84.559 103.839686) (width 0.2) (layer "F.Cu") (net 12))
 (segment (start 93.802 97.248943) (end 93.802 94.30424) (width 0.2) (layer "F.Cu") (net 12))
 (segment (start 84.559 105.000314) (end 84.559 104) (width 0.2) (layer "F.Cu") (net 12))
 (segment (start 90.050943 101) (end 93.802 97.248943) (width 0.2) (layer "F.Cu") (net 12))
 (segment (start 85.96 106.401314) (end 84.559 105.000314) (width 0.2) (layer "F.Cu") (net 12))
 (segment (start 91.03776 91.54) (end 90 91.54) (width 0.2) (layer "F.Cu") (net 12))
 (segment (start 81.011 103.069) (end 90 94.08) (width 0.2) (layer "F.Cu") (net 11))
 (segment (start 75.088686 124.42) (end 79.029686 128.361) (width 0.2) (layer "F.Cu") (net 11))
 (segment (start 63.96 124.42) (end 75.088686 124.42) (width 0.2) (layer "F.Cu") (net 11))
 (segment (start 80.190314 128.361) (end 81.011 127.540314) (width 0.2) (layer "F.Cu") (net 11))
 (segment (start 81.011 127.540314) (end 81.011 103.069) (width 0.2) (layer "F.Cu") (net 11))
 (segment (start 79.029686 128.361) (end 80.190314 128.361) (width 0.2) (layer "F.Cu") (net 11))
 (segment (start 74.75 94.08) (end 83.05424 94.08) (width 0.2) (layer "F.Cu") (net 8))
 (segment (start 89.28524 87.849) (end 92.47676 87.849) (width 0.2) (layer "F.Cu") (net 8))
 (segment (start 92.47676 87.849) (end 94.627 89.99924) (width 0.2) (layer "F.Cu") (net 8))
 (segment (start 78.894184 130.701) (end 65.945816 130.701) (width 0.2) (layer "F.Cu") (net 8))
 (segment (start 94.627 121.67453) (end 89.15253 127.149) (width 0.2) (layer "F.Cu") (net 8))
 (segment (start 82.446184 127.149) (end 78.894184 130.701) (width 0.2) (layer "F.Cu") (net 8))
 (segment (start 94.627 89.99924) (end 94.627 121.67453) (width 0.2) (layer "F.Cu") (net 8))
 (segment (start 62.559 127.314184) (end 62.559 117.941) (width 0.2) (layer "F.Cu") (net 8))
 (segment (start 65.945816 130.701) (end 62.559 127.314184) (width 0.2) (layer "F.Cu") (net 8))
 (segment (start 89.15253 127.149) (end 82.446184 127.149) (width 0.2) (layer "F.Cu") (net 8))
 (segment (start 62.559 117.941) (end 68.5 112) (width 0.2) (layer "F.Cu") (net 8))
 (segment (start 83.05424 94.08) (end 89.28524 87.849) (width 0.2) (layer "F.Cu") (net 8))
 (segment (start 73.75 94.12) (end 73.75 94.21) (width 0.2) (layer "B.Cu") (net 8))
 (segment (start 58.900001 91.647158) (end 57.899001 92.648158) (width 0.2) (layer "B.Cu") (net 14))
 (segment (start 57.899001 93.594652) (end 59.873349 95.569) (width 0.2) (layer "B.Cu") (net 14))
 (segment (start 75.811 95.569) (end 90 81.38) (width 0.2) (layer "B.Cu") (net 14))
 (segment (start 57.899001 92.648158) (end 57.899001 93.594652) (width 0.2) (layer "B.Cu") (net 14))
 (segment (start 59.873349 95.569) (end 75.811 95.569) (width 0.2) (layer "B.Cu") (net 14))
 (segment (start 54 107) (end 72 89) (width 0.2) (layer "F.Cu") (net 6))
 (segment (start 72 89) (end 74.75 89) (width 0.2) (layer "F.Cu") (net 6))
 (segment (start 90.76 97) (end 93.201 97) (width 0.2) (layer "F.Cu") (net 10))
 (segment (start 90.38 96.62) (end 90.5 96.5) (width 0.2) (layer "F.Cu") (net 10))
 (segment (start 93.161 97.04) (end 93.201 97) (width 0.2) (layer "F.Cu") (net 10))
 (segment (start 90 96.62) (end 90.38 96.62) (width 0.2) (layer "F.Cu") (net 10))
 (segment (start 90.5 96.5) (end 90.5 96.74) (width 0.2) (layer "F.Cu") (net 10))
 (segment (start 90.5 96.74) (end 90.76 97) (width 0.2) (layer "F.Cu") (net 10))
 (via (at 93.201 97) (size 0.6) (drill 0.3) (layers "F.Cu" "B.Cu") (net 10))
 (segment (start 93.201 97) (end 93.201 97.04) (width 0.2) (layer "B.Cu") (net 10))
 (segment (start 73.71224 91.54) (end 63.401 101.85124) (width 0.2) (layer "F.Cu") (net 7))
 (segment (start 63.401 105.201) (end 56.602 112) (width 0.2) (layer "F.Cu") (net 7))
 (segment (start 56.602 112) (end 54 112) (width 0.2) (layer "F.Cu") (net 7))
 (segment (start 63.401 101.85124) (end 63.401 105.201) (width 0.2) (layer "F.Cu") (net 7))
 (segment (start 74.75 91.54) (end 73.71224 91.54) (width 0.2) (layer "F.Cu") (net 7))
 (segment (start 64.100001 91.133661) (end 73.853662 81.38) (width 0.2) (layer "B.Cu") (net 3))
 (segment (start 73.853662 81.38) (end 74.75 81.38) (width 0.2) (layer "B.Cu") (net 3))
 (segment (start 64.100001 91.647158) (end 64.100001 91.133661) (width 0.2) (layer "B.Cu") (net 3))
 (segment (start 75.47676 86.479) (end 75.06388 86.06612) (width 0.2) (layer "B.Cu") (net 5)))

